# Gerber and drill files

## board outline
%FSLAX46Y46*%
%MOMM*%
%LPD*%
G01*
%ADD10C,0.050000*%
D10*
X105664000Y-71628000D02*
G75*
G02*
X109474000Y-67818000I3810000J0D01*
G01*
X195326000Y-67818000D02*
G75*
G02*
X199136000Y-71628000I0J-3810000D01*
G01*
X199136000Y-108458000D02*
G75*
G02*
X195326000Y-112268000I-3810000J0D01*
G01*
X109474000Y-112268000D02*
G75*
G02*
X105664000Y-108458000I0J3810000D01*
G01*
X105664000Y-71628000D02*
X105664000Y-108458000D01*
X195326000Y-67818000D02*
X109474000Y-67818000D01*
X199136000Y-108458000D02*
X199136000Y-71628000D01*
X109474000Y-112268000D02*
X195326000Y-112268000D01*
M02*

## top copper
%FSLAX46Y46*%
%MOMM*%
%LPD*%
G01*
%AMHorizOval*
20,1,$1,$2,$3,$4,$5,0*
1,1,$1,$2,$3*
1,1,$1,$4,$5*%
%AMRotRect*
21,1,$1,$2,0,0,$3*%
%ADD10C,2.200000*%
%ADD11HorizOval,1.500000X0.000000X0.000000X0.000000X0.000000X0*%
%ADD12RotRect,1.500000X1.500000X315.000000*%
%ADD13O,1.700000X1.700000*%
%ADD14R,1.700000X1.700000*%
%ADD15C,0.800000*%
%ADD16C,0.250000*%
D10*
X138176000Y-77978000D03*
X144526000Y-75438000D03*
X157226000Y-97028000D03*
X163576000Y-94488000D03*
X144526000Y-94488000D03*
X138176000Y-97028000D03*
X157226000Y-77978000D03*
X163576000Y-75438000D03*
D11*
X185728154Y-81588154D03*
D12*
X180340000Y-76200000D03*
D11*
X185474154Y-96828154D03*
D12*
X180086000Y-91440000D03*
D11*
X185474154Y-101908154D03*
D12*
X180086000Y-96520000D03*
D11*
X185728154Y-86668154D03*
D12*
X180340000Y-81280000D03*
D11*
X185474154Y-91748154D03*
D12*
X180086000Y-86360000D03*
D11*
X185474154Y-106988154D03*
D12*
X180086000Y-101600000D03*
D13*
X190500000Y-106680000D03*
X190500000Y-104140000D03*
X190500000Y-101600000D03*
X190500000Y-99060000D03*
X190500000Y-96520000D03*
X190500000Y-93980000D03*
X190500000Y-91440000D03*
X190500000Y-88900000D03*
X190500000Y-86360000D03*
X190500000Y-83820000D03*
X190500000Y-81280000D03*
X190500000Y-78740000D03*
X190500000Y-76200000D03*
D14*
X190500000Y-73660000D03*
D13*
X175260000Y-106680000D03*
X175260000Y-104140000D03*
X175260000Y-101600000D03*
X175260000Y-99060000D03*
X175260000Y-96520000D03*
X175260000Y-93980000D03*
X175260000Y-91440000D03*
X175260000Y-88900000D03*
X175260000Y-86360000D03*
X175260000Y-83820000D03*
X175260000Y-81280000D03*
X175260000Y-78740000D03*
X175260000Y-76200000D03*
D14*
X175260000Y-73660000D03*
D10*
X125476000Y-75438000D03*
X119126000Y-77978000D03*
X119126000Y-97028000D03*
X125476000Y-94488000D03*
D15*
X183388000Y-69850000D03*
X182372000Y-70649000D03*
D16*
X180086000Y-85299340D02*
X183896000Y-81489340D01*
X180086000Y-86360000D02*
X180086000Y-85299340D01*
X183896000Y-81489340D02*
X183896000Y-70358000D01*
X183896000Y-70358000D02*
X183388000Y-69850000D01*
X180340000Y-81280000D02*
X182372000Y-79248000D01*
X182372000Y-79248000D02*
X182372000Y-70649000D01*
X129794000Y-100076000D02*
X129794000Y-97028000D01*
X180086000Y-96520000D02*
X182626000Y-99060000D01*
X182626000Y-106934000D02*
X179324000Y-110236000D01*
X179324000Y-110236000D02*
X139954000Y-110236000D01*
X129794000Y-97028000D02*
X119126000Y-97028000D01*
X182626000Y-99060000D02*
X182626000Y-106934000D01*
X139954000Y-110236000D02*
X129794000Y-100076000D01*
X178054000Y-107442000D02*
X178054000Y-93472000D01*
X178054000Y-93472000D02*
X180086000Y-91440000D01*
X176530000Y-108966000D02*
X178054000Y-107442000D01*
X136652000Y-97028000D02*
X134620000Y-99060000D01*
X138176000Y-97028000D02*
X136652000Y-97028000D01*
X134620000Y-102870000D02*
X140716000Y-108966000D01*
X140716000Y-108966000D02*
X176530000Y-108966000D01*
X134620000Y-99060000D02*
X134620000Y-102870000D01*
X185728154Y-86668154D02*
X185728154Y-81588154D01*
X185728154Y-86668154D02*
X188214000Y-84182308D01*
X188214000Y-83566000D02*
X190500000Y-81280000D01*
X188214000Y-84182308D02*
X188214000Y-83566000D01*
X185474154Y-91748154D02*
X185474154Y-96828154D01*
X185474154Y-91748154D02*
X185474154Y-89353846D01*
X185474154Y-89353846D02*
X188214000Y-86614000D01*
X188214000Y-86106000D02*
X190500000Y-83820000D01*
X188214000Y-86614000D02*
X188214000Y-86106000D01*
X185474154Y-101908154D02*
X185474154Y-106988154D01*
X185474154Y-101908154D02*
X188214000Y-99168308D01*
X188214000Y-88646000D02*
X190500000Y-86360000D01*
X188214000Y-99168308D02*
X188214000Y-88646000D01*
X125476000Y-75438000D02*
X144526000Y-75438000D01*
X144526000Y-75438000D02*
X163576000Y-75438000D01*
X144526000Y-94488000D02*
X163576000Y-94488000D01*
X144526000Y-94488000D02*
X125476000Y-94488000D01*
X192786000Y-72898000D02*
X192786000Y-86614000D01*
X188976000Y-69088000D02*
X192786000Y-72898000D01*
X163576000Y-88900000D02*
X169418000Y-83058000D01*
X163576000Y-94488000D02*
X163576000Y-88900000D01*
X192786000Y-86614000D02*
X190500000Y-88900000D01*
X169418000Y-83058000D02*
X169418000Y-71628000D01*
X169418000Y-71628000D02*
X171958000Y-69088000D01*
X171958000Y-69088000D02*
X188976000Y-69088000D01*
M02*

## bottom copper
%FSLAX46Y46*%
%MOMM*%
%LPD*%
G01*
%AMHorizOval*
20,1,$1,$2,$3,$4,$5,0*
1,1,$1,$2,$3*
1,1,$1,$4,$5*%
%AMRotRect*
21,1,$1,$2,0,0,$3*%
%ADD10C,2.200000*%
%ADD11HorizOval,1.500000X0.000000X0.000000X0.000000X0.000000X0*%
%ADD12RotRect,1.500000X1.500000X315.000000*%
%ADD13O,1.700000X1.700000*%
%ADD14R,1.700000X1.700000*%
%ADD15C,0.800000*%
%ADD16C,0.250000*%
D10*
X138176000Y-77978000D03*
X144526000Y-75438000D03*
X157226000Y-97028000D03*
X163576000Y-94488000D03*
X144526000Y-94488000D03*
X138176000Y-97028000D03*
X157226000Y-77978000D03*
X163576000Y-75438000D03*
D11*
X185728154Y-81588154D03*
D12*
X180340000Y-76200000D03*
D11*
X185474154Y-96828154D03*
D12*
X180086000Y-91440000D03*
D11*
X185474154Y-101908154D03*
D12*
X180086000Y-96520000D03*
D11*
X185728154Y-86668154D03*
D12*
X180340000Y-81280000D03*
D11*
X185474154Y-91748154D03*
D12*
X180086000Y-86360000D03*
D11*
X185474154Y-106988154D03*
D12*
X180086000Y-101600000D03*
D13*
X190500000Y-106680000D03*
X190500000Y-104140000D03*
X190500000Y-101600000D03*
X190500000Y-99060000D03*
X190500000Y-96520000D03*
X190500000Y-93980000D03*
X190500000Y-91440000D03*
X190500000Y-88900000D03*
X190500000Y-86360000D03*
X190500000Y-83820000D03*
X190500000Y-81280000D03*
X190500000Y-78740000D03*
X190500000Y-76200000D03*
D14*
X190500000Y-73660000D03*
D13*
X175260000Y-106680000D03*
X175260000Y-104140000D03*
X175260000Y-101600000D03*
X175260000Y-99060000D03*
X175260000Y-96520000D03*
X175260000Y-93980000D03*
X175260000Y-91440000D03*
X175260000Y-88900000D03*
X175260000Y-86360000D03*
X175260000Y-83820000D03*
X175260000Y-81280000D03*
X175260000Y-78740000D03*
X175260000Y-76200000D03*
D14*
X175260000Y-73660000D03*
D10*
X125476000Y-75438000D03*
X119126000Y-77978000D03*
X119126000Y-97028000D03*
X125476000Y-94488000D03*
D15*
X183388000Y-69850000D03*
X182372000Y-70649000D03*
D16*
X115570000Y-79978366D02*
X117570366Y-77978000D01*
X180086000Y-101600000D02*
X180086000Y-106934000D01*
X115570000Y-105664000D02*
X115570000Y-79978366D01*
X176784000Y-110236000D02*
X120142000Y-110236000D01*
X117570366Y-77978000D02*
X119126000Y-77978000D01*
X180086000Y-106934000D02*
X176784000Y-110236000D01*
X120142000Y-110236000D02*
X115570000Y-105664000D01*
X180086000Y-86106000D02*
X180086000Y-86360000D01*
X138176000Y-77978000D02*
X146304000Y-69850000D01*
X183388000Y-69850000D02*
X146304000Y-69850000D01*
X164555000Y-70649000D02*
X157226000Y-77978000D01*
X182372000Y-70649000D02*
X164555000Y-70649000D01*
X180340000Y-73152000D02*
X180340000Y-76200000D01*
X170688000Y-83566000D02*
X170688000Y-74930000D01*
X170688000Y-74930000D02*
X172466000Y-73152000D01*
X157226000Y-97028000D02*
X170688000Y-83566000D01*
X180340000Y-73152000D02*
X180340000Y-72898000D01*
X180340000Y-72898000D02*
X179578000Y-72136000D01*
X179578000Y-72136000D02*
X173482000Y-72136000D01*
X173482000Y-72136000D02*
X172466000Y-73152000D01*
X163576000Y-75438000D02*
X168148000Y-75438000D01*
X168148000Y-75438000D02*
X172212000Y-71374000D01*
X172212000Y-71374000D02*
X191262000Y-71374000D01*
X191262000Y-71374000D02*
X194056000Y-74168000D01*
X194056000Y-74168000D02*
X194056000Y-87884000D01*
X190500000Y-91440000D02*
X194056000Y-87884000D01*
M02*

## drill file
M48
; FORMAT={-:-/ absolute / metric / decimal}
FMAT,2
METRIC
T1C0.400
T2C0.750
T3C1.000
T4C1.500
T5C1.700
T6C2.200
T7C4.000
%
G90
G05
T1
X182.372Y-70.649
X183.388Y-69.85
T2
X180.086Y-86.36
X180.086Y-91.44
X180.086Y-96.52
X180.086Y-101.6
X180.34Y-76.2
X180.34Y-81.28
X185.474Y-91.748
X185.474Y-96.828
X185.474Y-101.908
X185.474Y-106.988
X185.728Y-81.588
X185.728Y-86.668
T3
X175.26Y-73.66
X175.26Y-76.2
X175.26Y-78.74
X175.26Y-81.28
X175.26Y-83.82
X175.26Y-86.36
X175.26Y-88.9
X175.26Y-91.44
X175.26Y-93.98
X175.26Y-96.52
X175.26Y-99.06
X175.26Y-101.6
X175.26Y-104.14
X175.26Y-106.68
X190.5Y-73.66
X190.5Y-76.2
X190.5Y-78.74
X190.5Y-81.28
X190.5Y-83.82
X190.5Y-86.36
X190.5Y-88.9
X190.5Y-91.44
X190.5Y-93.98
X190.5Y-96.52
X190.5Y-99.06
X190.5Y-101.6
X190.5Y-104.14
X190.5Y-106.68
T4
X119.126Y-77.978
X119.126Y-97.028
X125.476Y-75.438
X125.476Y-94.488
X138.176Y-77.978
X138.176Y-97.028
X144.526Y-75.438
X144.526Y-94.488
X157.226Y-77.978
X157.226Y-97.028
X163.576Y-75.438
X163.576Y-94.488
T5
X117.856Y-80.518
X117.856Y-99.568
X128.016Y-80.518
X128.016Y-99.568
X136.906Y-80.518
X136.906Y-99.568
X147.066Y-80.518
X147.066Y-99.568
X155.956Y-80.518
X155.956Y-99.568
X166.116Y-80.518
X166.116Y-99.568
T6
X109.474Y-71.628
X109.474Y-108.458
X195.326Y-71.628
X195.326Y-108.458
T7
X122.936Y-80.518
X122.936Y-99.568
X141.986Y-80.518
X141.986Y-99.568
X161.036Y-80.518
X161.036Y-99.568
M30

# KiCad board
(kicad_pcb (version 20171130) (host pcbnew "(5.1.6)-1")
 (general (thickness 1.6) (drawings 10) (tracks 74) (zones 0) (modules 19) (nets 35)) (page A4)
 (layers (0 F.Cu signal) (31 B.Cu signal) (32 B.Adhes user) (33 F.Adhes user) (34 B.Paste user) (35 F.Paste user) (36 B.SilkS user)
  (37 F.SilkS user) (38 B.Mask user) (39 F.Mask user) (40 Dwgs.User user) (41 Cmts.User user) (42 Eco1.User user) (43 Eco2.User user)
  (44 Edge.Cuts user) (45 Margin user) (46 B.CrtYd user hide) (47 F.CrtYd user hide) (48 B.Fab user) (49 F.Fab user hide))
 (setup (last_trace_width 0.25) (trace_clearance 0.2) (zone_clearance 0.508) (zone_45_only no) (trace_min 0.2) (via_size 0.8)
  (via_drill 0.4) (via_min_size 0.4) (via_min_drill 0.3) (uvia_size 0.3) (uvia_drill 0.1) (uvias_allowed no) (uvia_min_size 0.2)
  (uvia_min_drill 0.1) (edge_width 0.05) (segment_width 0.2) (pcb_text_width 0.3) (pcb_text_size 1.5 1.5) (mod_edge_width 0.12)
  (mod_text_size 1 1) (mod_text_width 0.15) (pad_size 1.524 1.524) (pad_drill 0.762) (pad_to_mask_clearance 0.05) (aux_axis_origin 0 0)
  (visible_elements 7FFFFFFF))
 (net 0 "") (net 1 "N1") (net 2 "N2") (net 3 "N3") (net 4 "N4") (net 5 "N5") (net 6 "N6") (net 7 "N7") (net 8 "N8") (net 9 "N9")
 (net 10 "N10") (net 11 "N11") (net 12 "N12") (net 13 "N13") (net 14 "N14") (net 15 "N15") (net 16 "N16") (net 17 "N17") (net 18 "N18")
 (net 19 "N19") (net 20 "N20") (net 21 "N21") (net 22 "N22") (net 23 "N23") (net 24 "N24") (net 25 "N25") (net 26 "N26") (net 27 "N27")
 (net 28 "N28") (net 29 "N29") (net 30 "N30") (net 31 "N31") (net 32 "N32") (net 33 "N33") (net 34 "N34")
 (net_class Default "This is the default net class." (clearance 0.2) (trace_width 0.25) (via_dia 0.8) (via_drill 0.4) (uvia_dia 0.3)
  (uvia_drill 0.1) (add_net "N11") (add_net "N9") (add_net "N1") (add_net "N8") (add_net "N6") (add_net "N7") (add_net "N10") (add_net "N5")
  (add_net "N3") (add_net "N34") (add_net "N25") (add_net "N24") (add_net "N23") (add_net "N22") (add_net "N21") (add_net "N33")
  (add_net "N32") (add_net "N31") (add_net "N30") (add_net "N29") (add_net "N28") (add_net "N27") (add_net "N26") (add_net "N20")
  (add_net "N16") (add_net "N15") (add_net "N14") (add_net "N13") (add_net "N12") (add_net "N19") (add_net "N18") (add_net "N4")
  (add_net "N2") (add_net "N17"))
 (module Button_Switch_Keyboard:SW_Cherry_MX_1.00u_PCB (layer F.Cu) (at 144.526 75.438)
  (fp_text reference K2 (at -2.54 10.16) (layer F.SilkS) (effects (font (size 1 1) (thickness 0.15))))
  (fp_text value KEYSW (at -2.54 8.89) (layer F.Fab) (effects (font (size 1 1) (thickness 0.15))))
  (pad "" np_thru_hole circle (at 2.54 5.08) (size 1.7 1.7) (drill 1.7) (layers *.Cu *.Mask))
  (pad "" np_thru_hole circle (at -7.62 5.08) (size 1.7 1.7) (drill 1.7) (layers *.Cu *.Mask))
  (pad "" np_thru_hole circle (at -2.54 5.08) (size 4 4) (drill 4) (layers *.Cu *.Mask))
  (pad 2 thru_hole circle (at -6.35 2.54) (size 2.2 2.2) (drill 1.5) (layers *.Cu *.Mask) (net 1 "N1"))
  (pad 1 thru_hole circle (at 0 0) (size 2.2 2.2) (drill 1.5) (layers *.Cu *.Mask) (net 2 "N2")))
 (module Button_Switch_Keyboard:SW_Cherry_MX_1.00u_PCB (layer F.Cu) (at 163.576 94.488)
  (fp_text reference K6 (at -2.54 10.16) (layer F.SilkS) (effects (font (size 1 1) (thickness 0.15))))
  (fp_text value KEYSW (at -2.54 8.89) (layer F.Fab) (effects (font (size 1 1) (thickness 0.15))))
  (pad "" np_thru_hole circle (at 2.54 5.08) (size 1.7 1.7) (drill 1.7) (layers *.Cu *.Mask))
  (pad "" np_thru_hole circle (at -7.62 5.08) (size 1.7 1.7) (drill 1.7) (layers *.Cu *.Mask))
  (pad "" np_thru_hole circle (at -2.54 5.08) (size 4 4) (drill 4) (layers *.Cu *.Mask))
  (pad 2 thru_hole circle (at -6.35 2.54) (size 2.2 2.2) (drill 1.5) (layers *.Cu *.Mask) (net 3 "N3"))
  (pad 1 thru_hole circle (at 0 0) (size 2.2 2.2) (drill 1.5) (layers *.Cu *.Mask) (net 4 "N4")))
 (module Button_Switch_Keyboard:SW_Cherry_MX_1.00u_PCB (layer F.Cu) (at 144.526 94.488)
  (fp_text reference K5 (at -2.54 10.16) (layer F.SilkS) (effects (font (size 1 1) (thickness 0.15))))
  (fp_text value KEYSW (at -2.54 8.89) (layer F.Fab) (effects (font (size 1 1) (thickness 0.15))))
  (pad 1 thru_hole circle (at 0 0) (size 2.2 2.2) (drill 1.5) (layers *.Cu *.Mask) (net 4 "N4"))
  (pad 2 thru_hole circle (at -6.35 2.54) (size 2.2 2.2) (drill 1.5) (layers *.Cu *.Mask) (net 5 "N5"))
  (pad "" np_thru_hole circle (at -2.54 5.08) (size 4 4) (drill 4) (layers *.Cu *.Mask))
  (pad "" np_thru_hole circle (at -7.62 5.08) (size 1.7 1.7) (drill 1.7) (layers *.Cu *.Mask))
  (pad "" np_thru_hole circle (at 2.54 5.08) (size 1.7 1.7) (drill 1.7) (layers *.Cu *.Mask)))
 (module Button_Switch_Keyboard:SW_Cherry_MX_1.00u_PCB (layer F.Cu) (at 163.576 75.438)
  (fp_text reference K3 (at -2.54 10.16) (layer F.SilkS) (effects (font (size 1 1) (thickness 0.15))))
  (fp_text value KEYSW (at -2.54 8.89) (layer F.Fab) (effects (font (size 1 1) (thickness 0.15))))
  (pad "" np_thru_hole circle (at 2.54 5.08) (size 1.7 1.7) (drill 1.7) (layers *.Cu *.Mask))
  (pad "" np_thru_hole circle (at -7.62 5.08) (size 1.7 1.7) (drill 1.7) (layers *.Cu *.Mask))
  (pad "" np_thru_hole circle (at -2.54 5.08) (size 4 4) (drill 4) (layers *.Cu *.Mask))
  (pad 2 thru_hole circle (at -6.35 2.54) (size 2.2 2.2) (drill 1.5) (layers *.Cu *.Mask) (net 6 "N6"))
  (pad 1 thru_hole circle (at 0 0) (size 2.2 2.2) (drill 1.5) (layers *.Cu *.Mask) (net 2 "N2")))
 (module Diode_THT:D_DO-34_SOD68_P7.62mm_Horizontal (layer F.Cu) (at 180.34 76.2 315)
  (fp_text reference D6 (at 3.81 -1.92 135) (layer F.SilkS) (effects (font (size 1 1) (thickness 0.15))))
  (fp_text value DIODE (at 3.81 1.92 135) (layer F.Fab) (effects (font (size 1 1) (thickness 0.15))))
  (pad 2 thru_hole oval (at 7.62 0 315) (size 1.5 1.5) (drill 0.75) (layers *.Cu *.Mask) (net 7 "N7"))
  (pad 1 thru_hole rect (at 0 0 315) (size 1.5 1.5) (drill 0.75) (layers *.Cu *.Mask) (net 3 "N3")))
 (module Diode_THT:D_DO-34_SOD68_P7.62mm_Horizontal (layer F.Cu) (at 180.086 91.44 315)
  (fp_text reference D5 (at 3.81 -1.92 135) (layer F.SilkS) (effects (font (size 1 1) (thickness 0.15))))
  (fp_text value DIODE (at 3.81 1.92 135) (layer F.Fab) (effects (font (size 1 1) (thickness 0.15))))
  (pad 2 thru_hole oval (at 7.62 0 315) (size 1.5 1.5) (drill 0.75) (layers *.Cu *.Mask) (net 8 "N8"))
  (pad 1 thru_hole rect (at 0 0 315) (size 1.5 1.5) (drill 0.75) (layers *.Cu *.Mask) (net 5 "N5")))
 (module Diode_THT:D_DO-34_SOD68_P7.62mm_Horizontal (layer F.Cu) (at 180.086 96.52 315)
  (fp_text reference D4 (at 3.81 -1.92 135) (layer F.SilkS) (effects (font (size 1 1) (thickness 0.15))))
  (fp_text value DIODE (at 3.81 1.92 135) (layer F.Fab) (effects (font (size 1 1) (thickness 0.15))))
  (pad 2 thru_hole oval (at 7.62 0 315) (size 1.5 1.5) (drill 0.75) (layers *.Cu *.Mask) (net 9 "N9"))
  (pad 1 thru_hole rect (at 0 0 315) (size 1.5 1.5) (drill 0.75) (layers *.Cu *.Mask) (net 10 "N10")))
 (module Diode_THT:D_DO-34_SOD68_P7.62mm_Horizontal (layer F.Cu) (at 180.34 81.28 315)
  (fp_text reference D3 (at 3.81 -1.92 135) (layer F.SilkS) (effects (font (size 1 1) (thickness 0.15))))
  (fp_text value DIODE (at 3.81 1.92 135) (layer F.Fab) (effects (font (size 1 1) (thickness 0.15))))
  (pad 2 thru_hole oval (at 7.62 0 315) (size 1.5 1.5) (drill 0.75) (layers *.Cu *.Mask) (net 7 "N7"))
  (pad 1 thru_hole rect (at 0 0 315) (size 1.5 1.5) (drill 0.75) (layers *.Cu *.Mask) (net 6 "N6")))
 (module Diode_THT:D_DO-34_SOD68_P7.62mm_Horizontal (layer F.Cu) (at 180.086 86.36 315)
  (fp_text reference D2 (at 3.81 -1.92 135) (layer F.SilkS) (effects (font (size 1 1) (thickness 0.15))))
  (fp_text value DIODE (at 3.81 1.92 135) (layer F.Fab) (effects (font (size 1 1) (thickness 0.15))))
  (pad 2 thru_hole oval (at 7.62 0 315) (size 1.5 1.5) (drill 0.75) (layers *.Cu *.Mask) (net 8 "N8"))
  (pad 1 thru_hole rect (at 0 0 315) (size 1.5 1.5) (drill 0.75) (layers *.Cu *.Mask) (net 1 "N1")))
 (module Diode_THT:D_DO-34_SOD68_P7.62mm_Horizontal (layer F.Cu) (at 180.086 101.6 315)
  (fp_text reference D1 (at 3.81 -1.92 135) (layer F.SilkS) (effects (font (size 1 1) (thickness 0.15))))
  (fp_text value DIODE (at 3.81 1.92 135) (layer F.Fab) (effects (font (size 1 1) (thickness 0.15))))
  (pad 2 thru_hole oval (at 7.62 0 315) (size 1.5 1.5) (drill 0.75) (layers *.Cu *.Mask) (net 9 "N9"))
  (pad 1 thru_hole rect (at 0 0 315) (size 1.5 1.5) (drill 0.75) (layers *.Cu *.Mask) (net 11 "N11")))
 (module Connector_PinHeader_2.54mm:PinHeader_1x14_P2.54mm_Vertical (layer F.Cu) (at 190.5 73.66)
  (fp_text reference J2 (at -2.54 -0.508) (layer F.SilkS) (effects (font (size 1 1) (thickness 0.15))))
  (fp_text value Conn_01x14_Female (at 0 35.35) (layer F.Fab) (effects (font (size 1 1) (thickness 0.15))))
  (pad 14 thru_hole oval (at 0 33.02) (size 1.7 1.7) (drill 1) (layers *.Cu *.Mask) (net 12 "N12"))
  (pad 13 thru_hole oval (at 0 30.48) (size 1.7 1.7) (drill 1) (layers *.Cu *.Mask) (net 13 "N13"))
  (pad 12 thru_hole oval (at 0 27.94) (size 1.7 1.7) (drill 1) (layers *.Cu *.Mask) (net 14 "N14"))
  (pad 11 thru_hole oval (at 0 25.4) (size 1.7 1.7) (drill 1) (layers *.Cu *.Mask) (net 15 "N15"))
  (pad 10 thru_hole oval (at 0 22.86) (size 1.7 1.7) (drill 1) (layers *.Cu *.Mask) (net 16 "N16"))
  (pad 9 thru_hole oval (at 0 20.32) (size 1.7 1.7) (drill 1) (layers *.Cu *.Mask) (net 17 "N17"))
  (pad 8 thru_hole oval (at 0 17.78) (size 1.7 1.7) (drill 1) (layers *.Cu *.Mask) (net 2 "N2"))
  (pad 7 thru_hole oval (at 0 15.24) (size 1.7 1.7) (drill 1) (layers *.Cu *.Mask) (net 4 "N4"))
  (pad 6 thru_hole oval (at 0 12.7) (size 1.7 1.7) (drill 1) (layers *.Cu *.Mask) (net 9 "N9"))
  (pad 5 thru_hole oval (at 0 10.16) (size 1.7 1.7) (drill 1) (layers *.Cu *.Mask) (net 8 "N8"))
  (pad 4 thru_hole oval (at 0 7.62) (size 1.7 1.7) (drill 1) (layers *.Cu *.Mask) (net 7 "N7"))
  (pad 3 thru_hole oval (at 0 5.08) (size 1.7 1.7) (drill 1) (layers *.Cu *.Mask) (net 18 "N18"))
  (pad 2 thru_hole oval (at 0 2.54) (size 1.7 1.7) (drill 1) (layers *.Cu *.Mask) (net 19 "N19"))
  (pad 1 thru_hole rect (at 0 0) (size 1.7 1.7) (drill 1) (layers *.Cu *.Mask) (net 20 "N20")))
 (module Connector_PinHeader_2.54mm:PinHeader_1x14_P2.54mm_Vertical (layer F.Cu) (at 175.26 73.66)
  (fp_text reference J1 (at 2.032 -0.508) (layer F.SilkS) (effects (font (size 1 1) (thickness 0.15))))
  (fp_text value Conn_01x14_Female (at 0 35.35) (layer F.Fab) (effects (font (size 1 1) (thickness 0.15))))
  (pad 14 thru_hole oval (at 0 33.02) (size 1.7 1.7) (drill 1) (layers *.Cu *.Mask) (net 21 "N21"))
  (pad 13 thru_hole oval (at 0 30.48) (size 1.7 1.7) (drill 1) (layers *.Cu *.Mask) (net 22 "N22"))
  (pad 12 thru_hole oval (at 0 27.94) (size 1.7 1.7) (drill 1) (layers *.Cu *.Mask) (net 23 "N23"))
  (pad 11 thru_hole oval (at 0 25.4) (size 1.7 1.7) (drill 1) (layers *.Cu *.Mask) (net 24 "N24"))
  (pad 10 thru_hole oval (at 0 22.86) (size 1.7 1.7) (drill 1) (layers *.Cu *.Mask) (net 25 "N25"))
  (pad 9 thru_hole oval (at 0 20.32) (size 1.7 1.7) (drill 1) (layers *.Cu *.Mask) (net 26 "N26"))
  (pad 8 thru_hole oval (at 0 17.78) (size 1.7 1.7) (drill 1) (layers *.Cu *.Mask) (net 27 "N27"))
  (pad 7 thru_hole oval (at 0 15.24) (size 1.7 1.7) (drill 1) (layers *.Cu *.Mask) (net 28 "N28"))
  (pad 6 thru_hole oval (at 0 12.7) (size 1.7 1.7) (drill 1) (layers *.Cu *.Mask) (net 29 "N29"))
  (pad 5 thru_hole oval (at 0 10.16) (size 1.7 1.7) (drill 1) (layers *.Cu *.Mask) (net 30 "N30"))
  (pad 4 thru_hole oval (at 0 7.62) (size 1.7 1.7) (drill 1) (layers *.Cu *.Mask) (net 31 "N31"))
  (pad 3 thru_hole oval (at 0 5.08) (size 1.7 1.7) (drill 1) (layers *.Cu *.Mask) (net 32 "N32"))
  (pad 2 thru_hole oval (at 0 2.54) (size 1.7 1.7) (drill 1) (layers *.Cu *.Mask) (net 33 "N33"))
  (pad 1 thru_hole rect (at 0 0) (size 1.7 1.7) (drill 1) (layers *.Cu *.Mask) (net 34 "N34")))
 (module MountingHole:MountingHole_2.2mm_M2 (layer F.Cu) (at 109.474 71.628)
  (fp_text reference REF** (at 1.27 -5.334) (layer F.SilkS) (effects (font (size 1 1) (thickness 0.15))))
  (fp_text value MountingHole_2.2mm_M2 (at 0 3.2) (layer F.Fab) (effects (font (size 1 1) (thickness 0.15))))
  (pad 1 np_thru_hole circle (at 0 0) (size 2.2 2.2) (drill 2.2) (layers *.Cu *.Mask)))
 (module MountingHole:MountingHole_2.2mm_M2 (layer F.Cu) (at 109.474 108.458)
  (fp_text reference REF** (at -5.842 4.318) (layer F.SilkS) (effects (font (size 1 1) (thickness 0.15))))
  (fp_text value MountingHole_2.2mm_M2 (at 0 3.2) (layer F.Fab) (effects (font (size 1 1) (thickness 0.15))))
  (pad 1 np_thru_hole circle (at 0 0) (size 2.2 2.2) (drill 2.2) (layers *.Cu *.Mask)))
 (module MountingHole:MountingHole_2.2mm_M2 (layer F.Cu) (at 195.326 108.458)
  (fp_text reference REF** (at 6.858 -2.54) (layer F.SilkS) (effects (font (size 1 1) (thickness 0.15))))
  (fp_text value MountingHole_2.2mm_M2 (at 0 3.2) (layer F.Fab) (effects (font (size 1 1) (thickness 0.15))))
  (pad 1 np_thru_hole circle (at 0 0) (size 2.2 2.2) (drill 2.2) (layers *.Cu *.Mask)))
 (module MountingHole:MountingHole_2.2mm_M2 (layer F.Cu) (at 195.326 71.628)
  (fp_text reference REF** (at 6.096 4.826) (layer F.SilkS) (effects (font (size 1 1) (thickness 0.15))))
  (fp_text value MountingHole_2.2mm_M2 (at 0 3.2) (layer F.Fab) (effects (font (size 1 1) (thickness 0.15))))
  (pad 1 np_thru_hole circle (at 0 0) (size 2.2 2.2) (drill 2.2) (layers *.Cu *.Mask)))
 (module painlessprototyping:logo (layer B.Cu) (at 167.386 88.646 180)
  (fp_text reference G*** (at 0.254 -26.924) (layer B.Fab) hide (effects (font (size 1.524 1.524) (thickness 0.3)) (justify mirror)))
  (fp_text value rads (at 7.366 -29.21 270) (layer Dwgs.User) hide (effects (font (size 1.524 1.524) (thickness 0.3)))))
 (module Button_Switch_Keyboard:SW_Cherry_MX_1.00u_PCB (layer F.Cu) (at 125.476 75.438)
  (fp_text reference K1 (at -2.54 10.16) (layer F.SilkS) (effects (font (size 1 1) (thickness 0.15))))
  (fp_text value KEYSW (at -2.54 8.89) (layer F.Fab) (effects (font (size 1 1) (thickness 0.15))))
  (pad 1 thru_hole circle (at 0 0) (size 2.2 2.2) (drill 1.5) (layers *.Cu *.Mask) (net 2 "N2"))
  (pad 2 thru_hole circle (at -6.35 2.54) (size 2.2 2.2) (drill 1.5) (layers *.Cu *.Mask) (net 11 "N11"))
  (pad "" np_thru_hole circle (at -2.54 5.08) (size 4 4) (drill 4) (layers *.Cu *.Mask))
  (pad "" np_thru_hole circle (at -7.62 5.08) (size 1.7 1.7) (drill 1.7) (layers *.Cu *.Mask))
  (pad "" np_thru_hole circle (at 2.54 5.08) (size 1.7 1.7) (drill 1.7) (layers *.Cu *.Mask)))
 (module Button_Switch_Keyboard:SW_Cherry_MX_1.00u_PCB (layer F.Cu) (at 125.476 94.488)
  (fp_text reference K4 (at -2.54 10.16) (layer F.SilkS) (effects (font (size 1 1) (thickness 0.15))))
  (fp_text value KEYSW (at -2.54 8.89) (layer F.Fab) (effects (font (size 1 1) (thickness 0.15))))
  (pad "" np_thru_hole circle (at 2.54 5.08) (size 1.7 1.7) (drill 1.7) (layers *.Cu *.Mask))
  (pad "" np_thru_hole circle (at -7.62 5.08) (size 1.7 1.7) (drill 1.7) (layers *.Cu *.Mask))
  (pad "" np_thru_hole circle (at -2.54 5.08) (size 4 4) (drill 4) (layers *.Cu *.Mask))
  (pad 2 thru_hole circle (at -6.35 2.54) (size 2.2 2.2) (drill 1.5) (layers *.Cu *.Mask) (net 10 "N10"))
  (pad 1 thru_hole circle (at 0 0) (size 2.2 2.2) (drill 1.5) (layers *.Cu *.Mask) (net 4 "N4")))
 (gr_arc (start 109.474 71.628) (end 109.474 67.818) (angle -90) (layer Edge.Cuts) (width 0.05))
 (gr_arc (start 195.326 71.628) (end 199.136 71.628) (angle -90) (layer Edge.Cuts) (width 0.05))
 (gr_arc (start 195.326 108.458) (end 195.326 112.268) (angle -90) (layer Edge.Cuts) (width 0.05))
 (gr_arc (start 109.474 108.458) (end 105.664 108.458) (angle -90) (layer Edge.Cuts) (width 0.05))
 (gr_line (start 105.664 71.628) (end 105.664 108.458) (layer Edge.Cuts) (width 0.05))
 (gr_line (start 195.326 67.818) (end 109.474 67.818) (layer Edge.Cuts) (width 0.05))
 (gr_line (start 199.136 108.458) (end 199.136 71.628) (layer Edge.Cuts) (width 0.05))
 (gr_line (start 109.474 112.268) (end 195.326 112.268) (layer Edge.Cuts) (width 0.05))
 (segment (start 115.57 79.978366) (end 117.570366 77.978) (width 0.25) (layer B.Cu) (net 11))
 (segment (start 180.086 101.6) (end 180.086 106.934) (width 0.25) (layer B.Cu) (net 11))
 (segment (start 115.57 105.664) (end 115.57 79.978366) (width 0.25) (layer B.Cu) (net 11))
 (segment (start 176.784 110.236) (end 120.142 110.236) (width 0.25) (layer B.Cu) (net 11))
 (segment (start 117.570366 77.978) (end 119.126 77.978) (width 0.25) (layer B.Cu) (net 11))
 (segment (start 180.086 106.934) (end 176.784 110.236) (width 0.25) (layer B.Cu) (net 11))
 (segment (start 120.142 110.236) (end 115.57 105.664) (width 0.25) (layer B.Cu) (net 11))
 (segment (start 180.086 86.106) (end 180.086 86.36) (width 0.25) (layer B.Cu) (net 1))
 (segment (start 138.176 77.978) (end 146.304 69.85) (width 0.25) (layer B.Cu) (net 1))
 (segment (start 180.086 85.29934) (end 183.896 81.48934) (width 0.25) (layer F.Cu) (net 1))
 (segment (start 180.086 86.36) (end 180.086 85.29934) (width 0.25) (layer F.Cu) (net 1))
 (via (at 183.388 69.85) (size 0.8) (drill 0.4) (layers F.Cu B.Cu) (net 1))
 (segment (start 183.896 81.48934) (end 183.896 70.358) (width 0.25) (layer F.Cu) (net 1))
 (segment (start 183.896 70.358) (end 183.388 69.85) (width 0.25) (layer F.Cu) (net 1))
 (segment (start 183.388 69.85) (end 146.304 69.85) (width 0.25) (layer B.Cu) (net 1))
 (via (at 182.372 70.649) (size 0.8) (drill 0.4) (layers F.Cu B.Cu) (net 6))
 (segment (start 180.34 81.28) (end 182.372 79.248) (width 0.25) (layer F.Cu) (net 6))
 (segment (start 182.372 79.248) (end 182.372 70.649) (width 0.25) (layer F.Cu) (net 6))
 (segment (start 164.555 70.649) (end 157.226 77.978) (width 0.25) (layer B.Cu) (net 6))
 (segment (start 182.372 70.649) (end 164.555 70.649) (width 0.25) (layer B.Cu) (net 6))
 (segment (start 129.794 100.076) (end 129.794 97.028) (width 0.25) (layer F.Cu) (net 10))
 (segment (start 180.086 96.52) (end 182.626 99.06) (width 0.25) (layer F.Cu) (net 10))
 (segment (start 182.626 106.934) (end 179.324 110.236) (width 0.25) (layer F.Cu) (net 10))
 (segment (start 179.324 110.236) (end 139.954 110.236) (width 0.25) (layer F.Cu) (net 10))
 (segment (start 129.794 97.028) (end 119.126 97.028) (width 0.25) (layer F.Cu) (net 10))
 (segment (start 182.626 99.06) (end 182.626 106.934) (width 0.25) (layer F.Cu) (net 10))
 (segment (start 139.954 110.236) (end 129.794 100.076) (width 0.25) (layer F.Cu) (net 10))
 (segment (start 178.054 107.442) (end 178.054 93.472) (width 0.25) (layer F.Cu) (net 5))
 (segment (start 178.054 93.472) (end 180.086 91.44) (width 0.25) (layer F.Cu) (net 5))
 (segment (start 176.53 108.966) (end 178.054 107.442) (width 0.25) (layer F.Cu) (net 5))
 (segment (start 136.652 97.028) (end 134.62 99.06) (width 0.25) (layer F.Cu) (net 5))
 (segment (start 138.176 97.028) (end 136.652 97.028) (width 0.25) (layer F.Cu) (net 5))
 (segment (start 134.62 102.87) (end 140.716 108.966) (width 0.25) (layer F.Cu) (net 5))
 (segment (start 140.716 108.966) (end 176.53 108.966) (width 0.25) (layer F.Cu) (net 5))
 (segment (start 134.62 99.06) (end 134.62 102.87) (width 0.25) (layer F.Cu) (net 5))
 (segment (start 180.34 73.152) (end 180.34 76.2) (width 0.25) (layer B.Cu) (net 3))
 (segment (start 170.688 83.566) (end 170.688 74.93) (width 0.25) (layer B.Cu) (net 3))
 (segment (start 170.688 74.93) (end 172.466 73.152) (width 0.25) (layer B.Cu) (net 3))
 (segment (start 157.226 97.028) (end 170.688 83.566) (width 0.25) (layer B.Cu) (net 3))
 (segment (start 180.34 73.152) (end 180.34 72.898) (width 0.25) (layer B.Cu) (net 3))
 (segment (start 180.34 72.898) (end 179.578 72.136) (width 0.25) (layer B.Cu) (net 3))
 (segment (start 179.578 72.136) (end 173.482 72.136) (width 0.25) (layer B.Cu) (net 3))
 (segment (start 173.482 72.136) (end 172.466 73.152) (width 0.25) (layer B.Cu) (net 3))
 (segment (start 185.728154 86.668154) (end 185.728154 81.588154) (width 0.25) (layer F.Cu) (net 7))
 (segment (start 185.728154 86.668154) (end 188.214 84.182308) (width 0.25) (layer F.Cu) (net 7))
 (segment (start 188.214 83.566) (end 190.5 81.28) (width 0.25) (layer F.Cu) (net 7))
 (segment (start 188.214 84.182308) (end 188.214 83.566) (width 0.25) (layer F.Cu) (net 7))
 (segment (start 185.474154 91.748154) (end 185.474154 96.828154) (width 0.25) (layer F.Cu) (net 8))
 (segment (start 185.474154 91.748154) (end 185.474154 89.353846) (width 0.25) (layer F.Cu) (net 8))
 (segment (start 185.474154 89.353846) (end 188.214 86.614) (width 0.25) (layer F.Cu) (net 8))
 (segment (start 188.214 86.106) (end 190.5 83.82) (width 0.25) (layer F.Cu) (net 8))
 (segment (start 188.214 86.614) (end 188.214 86.106) (width 0.25) (layer F.Cu) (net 8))
 (segment (start 185.474154 101.908154) (end 185.474154 106.988154) (width 0.25) (layer F.Cu) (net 9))
 (segment (start 185.474154 101.908154) (end 188.214 99.168308) (width 0.25) (layer F.Cu) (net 9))
 (segment (start 188.214 88.646) (end 190.5 86.36) (width 0.25) (layer F.Cu) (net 9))
 (segment (start 188.214 99.168308) (end 188.214 88.646) (width 0.25) (layer F.Cu) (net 9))
 (segment (start 125.476 75.438) (end 144.526 75.438) (width 0.25) (layer F.Cu) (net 2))
 (segment (start 144.526 75.438) (end 163.576 75.438) (width 0.25) (layer F.Cu) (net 2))
 (segment (start 163.576 75.438) (end 168.148 75.438) (width 0.25) (layer B.Cu) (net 2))
 (segment (start 168.148 75.438) (end 172.212 71.374) (width 0.25) (layer B.Cu) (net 2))
 (segment (start 172.212 71.374) (end 191.262 71.374) (width 0.25) (layer B.Cu) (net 2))
 (segment (start 191.262 71.374) (end 194.056 74.168) (width 0.25) (layer B.Cu) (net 2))
 (segment (start 194.056 74.168) (end 194.056 87.884) (width 0.25) (layer B.Cu) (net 2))
 (segment (start 190.5 91.44) (end 194.056 87.884) (width 0.25) (layer B.Cu) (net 2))
 (segment (start 144.526 94.488) (end 163.576 94.488) (width 0.25) (layer F.Cu) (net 4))
 (segment (start 144.526 94.488) (end 125.476 94.488) (width 0.25) (layer F.Cu) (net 4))
 (segment (start 192.786 72.898) (end 192.786 86.614) (width 0.25) (layer F.Cu) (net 4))
 (segment (start 188.976 69.088) (end 192.786 72.898) (width 0.25) (layer F.Cu) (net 4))
 (segment (start 163.576 88.9) (end 169.418 83.058) (width 0.25) (layer F.Cu) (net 4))
 (segment (start 163.576 94.488) (end 163.576 88.9) (width 0.25) (layer F.Cu) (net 4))
 (segment (start 192.786 86.614) (end 190.5 88.9) (width 0.25) (layer F.Cu) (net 4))
 (segment (start 169.418 83.058) (end 169.418 71.628) (width 0.25) (layer F.Cu) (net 4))
 (segment (start 169.418 71.628) (end 171.958 69.088) (width 0.25) (layer F.Cu) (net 4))
 (segment (start 171.958 69.088) (end 188.976 69.088) (width 0.25) (layer F.Cu) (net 4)))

